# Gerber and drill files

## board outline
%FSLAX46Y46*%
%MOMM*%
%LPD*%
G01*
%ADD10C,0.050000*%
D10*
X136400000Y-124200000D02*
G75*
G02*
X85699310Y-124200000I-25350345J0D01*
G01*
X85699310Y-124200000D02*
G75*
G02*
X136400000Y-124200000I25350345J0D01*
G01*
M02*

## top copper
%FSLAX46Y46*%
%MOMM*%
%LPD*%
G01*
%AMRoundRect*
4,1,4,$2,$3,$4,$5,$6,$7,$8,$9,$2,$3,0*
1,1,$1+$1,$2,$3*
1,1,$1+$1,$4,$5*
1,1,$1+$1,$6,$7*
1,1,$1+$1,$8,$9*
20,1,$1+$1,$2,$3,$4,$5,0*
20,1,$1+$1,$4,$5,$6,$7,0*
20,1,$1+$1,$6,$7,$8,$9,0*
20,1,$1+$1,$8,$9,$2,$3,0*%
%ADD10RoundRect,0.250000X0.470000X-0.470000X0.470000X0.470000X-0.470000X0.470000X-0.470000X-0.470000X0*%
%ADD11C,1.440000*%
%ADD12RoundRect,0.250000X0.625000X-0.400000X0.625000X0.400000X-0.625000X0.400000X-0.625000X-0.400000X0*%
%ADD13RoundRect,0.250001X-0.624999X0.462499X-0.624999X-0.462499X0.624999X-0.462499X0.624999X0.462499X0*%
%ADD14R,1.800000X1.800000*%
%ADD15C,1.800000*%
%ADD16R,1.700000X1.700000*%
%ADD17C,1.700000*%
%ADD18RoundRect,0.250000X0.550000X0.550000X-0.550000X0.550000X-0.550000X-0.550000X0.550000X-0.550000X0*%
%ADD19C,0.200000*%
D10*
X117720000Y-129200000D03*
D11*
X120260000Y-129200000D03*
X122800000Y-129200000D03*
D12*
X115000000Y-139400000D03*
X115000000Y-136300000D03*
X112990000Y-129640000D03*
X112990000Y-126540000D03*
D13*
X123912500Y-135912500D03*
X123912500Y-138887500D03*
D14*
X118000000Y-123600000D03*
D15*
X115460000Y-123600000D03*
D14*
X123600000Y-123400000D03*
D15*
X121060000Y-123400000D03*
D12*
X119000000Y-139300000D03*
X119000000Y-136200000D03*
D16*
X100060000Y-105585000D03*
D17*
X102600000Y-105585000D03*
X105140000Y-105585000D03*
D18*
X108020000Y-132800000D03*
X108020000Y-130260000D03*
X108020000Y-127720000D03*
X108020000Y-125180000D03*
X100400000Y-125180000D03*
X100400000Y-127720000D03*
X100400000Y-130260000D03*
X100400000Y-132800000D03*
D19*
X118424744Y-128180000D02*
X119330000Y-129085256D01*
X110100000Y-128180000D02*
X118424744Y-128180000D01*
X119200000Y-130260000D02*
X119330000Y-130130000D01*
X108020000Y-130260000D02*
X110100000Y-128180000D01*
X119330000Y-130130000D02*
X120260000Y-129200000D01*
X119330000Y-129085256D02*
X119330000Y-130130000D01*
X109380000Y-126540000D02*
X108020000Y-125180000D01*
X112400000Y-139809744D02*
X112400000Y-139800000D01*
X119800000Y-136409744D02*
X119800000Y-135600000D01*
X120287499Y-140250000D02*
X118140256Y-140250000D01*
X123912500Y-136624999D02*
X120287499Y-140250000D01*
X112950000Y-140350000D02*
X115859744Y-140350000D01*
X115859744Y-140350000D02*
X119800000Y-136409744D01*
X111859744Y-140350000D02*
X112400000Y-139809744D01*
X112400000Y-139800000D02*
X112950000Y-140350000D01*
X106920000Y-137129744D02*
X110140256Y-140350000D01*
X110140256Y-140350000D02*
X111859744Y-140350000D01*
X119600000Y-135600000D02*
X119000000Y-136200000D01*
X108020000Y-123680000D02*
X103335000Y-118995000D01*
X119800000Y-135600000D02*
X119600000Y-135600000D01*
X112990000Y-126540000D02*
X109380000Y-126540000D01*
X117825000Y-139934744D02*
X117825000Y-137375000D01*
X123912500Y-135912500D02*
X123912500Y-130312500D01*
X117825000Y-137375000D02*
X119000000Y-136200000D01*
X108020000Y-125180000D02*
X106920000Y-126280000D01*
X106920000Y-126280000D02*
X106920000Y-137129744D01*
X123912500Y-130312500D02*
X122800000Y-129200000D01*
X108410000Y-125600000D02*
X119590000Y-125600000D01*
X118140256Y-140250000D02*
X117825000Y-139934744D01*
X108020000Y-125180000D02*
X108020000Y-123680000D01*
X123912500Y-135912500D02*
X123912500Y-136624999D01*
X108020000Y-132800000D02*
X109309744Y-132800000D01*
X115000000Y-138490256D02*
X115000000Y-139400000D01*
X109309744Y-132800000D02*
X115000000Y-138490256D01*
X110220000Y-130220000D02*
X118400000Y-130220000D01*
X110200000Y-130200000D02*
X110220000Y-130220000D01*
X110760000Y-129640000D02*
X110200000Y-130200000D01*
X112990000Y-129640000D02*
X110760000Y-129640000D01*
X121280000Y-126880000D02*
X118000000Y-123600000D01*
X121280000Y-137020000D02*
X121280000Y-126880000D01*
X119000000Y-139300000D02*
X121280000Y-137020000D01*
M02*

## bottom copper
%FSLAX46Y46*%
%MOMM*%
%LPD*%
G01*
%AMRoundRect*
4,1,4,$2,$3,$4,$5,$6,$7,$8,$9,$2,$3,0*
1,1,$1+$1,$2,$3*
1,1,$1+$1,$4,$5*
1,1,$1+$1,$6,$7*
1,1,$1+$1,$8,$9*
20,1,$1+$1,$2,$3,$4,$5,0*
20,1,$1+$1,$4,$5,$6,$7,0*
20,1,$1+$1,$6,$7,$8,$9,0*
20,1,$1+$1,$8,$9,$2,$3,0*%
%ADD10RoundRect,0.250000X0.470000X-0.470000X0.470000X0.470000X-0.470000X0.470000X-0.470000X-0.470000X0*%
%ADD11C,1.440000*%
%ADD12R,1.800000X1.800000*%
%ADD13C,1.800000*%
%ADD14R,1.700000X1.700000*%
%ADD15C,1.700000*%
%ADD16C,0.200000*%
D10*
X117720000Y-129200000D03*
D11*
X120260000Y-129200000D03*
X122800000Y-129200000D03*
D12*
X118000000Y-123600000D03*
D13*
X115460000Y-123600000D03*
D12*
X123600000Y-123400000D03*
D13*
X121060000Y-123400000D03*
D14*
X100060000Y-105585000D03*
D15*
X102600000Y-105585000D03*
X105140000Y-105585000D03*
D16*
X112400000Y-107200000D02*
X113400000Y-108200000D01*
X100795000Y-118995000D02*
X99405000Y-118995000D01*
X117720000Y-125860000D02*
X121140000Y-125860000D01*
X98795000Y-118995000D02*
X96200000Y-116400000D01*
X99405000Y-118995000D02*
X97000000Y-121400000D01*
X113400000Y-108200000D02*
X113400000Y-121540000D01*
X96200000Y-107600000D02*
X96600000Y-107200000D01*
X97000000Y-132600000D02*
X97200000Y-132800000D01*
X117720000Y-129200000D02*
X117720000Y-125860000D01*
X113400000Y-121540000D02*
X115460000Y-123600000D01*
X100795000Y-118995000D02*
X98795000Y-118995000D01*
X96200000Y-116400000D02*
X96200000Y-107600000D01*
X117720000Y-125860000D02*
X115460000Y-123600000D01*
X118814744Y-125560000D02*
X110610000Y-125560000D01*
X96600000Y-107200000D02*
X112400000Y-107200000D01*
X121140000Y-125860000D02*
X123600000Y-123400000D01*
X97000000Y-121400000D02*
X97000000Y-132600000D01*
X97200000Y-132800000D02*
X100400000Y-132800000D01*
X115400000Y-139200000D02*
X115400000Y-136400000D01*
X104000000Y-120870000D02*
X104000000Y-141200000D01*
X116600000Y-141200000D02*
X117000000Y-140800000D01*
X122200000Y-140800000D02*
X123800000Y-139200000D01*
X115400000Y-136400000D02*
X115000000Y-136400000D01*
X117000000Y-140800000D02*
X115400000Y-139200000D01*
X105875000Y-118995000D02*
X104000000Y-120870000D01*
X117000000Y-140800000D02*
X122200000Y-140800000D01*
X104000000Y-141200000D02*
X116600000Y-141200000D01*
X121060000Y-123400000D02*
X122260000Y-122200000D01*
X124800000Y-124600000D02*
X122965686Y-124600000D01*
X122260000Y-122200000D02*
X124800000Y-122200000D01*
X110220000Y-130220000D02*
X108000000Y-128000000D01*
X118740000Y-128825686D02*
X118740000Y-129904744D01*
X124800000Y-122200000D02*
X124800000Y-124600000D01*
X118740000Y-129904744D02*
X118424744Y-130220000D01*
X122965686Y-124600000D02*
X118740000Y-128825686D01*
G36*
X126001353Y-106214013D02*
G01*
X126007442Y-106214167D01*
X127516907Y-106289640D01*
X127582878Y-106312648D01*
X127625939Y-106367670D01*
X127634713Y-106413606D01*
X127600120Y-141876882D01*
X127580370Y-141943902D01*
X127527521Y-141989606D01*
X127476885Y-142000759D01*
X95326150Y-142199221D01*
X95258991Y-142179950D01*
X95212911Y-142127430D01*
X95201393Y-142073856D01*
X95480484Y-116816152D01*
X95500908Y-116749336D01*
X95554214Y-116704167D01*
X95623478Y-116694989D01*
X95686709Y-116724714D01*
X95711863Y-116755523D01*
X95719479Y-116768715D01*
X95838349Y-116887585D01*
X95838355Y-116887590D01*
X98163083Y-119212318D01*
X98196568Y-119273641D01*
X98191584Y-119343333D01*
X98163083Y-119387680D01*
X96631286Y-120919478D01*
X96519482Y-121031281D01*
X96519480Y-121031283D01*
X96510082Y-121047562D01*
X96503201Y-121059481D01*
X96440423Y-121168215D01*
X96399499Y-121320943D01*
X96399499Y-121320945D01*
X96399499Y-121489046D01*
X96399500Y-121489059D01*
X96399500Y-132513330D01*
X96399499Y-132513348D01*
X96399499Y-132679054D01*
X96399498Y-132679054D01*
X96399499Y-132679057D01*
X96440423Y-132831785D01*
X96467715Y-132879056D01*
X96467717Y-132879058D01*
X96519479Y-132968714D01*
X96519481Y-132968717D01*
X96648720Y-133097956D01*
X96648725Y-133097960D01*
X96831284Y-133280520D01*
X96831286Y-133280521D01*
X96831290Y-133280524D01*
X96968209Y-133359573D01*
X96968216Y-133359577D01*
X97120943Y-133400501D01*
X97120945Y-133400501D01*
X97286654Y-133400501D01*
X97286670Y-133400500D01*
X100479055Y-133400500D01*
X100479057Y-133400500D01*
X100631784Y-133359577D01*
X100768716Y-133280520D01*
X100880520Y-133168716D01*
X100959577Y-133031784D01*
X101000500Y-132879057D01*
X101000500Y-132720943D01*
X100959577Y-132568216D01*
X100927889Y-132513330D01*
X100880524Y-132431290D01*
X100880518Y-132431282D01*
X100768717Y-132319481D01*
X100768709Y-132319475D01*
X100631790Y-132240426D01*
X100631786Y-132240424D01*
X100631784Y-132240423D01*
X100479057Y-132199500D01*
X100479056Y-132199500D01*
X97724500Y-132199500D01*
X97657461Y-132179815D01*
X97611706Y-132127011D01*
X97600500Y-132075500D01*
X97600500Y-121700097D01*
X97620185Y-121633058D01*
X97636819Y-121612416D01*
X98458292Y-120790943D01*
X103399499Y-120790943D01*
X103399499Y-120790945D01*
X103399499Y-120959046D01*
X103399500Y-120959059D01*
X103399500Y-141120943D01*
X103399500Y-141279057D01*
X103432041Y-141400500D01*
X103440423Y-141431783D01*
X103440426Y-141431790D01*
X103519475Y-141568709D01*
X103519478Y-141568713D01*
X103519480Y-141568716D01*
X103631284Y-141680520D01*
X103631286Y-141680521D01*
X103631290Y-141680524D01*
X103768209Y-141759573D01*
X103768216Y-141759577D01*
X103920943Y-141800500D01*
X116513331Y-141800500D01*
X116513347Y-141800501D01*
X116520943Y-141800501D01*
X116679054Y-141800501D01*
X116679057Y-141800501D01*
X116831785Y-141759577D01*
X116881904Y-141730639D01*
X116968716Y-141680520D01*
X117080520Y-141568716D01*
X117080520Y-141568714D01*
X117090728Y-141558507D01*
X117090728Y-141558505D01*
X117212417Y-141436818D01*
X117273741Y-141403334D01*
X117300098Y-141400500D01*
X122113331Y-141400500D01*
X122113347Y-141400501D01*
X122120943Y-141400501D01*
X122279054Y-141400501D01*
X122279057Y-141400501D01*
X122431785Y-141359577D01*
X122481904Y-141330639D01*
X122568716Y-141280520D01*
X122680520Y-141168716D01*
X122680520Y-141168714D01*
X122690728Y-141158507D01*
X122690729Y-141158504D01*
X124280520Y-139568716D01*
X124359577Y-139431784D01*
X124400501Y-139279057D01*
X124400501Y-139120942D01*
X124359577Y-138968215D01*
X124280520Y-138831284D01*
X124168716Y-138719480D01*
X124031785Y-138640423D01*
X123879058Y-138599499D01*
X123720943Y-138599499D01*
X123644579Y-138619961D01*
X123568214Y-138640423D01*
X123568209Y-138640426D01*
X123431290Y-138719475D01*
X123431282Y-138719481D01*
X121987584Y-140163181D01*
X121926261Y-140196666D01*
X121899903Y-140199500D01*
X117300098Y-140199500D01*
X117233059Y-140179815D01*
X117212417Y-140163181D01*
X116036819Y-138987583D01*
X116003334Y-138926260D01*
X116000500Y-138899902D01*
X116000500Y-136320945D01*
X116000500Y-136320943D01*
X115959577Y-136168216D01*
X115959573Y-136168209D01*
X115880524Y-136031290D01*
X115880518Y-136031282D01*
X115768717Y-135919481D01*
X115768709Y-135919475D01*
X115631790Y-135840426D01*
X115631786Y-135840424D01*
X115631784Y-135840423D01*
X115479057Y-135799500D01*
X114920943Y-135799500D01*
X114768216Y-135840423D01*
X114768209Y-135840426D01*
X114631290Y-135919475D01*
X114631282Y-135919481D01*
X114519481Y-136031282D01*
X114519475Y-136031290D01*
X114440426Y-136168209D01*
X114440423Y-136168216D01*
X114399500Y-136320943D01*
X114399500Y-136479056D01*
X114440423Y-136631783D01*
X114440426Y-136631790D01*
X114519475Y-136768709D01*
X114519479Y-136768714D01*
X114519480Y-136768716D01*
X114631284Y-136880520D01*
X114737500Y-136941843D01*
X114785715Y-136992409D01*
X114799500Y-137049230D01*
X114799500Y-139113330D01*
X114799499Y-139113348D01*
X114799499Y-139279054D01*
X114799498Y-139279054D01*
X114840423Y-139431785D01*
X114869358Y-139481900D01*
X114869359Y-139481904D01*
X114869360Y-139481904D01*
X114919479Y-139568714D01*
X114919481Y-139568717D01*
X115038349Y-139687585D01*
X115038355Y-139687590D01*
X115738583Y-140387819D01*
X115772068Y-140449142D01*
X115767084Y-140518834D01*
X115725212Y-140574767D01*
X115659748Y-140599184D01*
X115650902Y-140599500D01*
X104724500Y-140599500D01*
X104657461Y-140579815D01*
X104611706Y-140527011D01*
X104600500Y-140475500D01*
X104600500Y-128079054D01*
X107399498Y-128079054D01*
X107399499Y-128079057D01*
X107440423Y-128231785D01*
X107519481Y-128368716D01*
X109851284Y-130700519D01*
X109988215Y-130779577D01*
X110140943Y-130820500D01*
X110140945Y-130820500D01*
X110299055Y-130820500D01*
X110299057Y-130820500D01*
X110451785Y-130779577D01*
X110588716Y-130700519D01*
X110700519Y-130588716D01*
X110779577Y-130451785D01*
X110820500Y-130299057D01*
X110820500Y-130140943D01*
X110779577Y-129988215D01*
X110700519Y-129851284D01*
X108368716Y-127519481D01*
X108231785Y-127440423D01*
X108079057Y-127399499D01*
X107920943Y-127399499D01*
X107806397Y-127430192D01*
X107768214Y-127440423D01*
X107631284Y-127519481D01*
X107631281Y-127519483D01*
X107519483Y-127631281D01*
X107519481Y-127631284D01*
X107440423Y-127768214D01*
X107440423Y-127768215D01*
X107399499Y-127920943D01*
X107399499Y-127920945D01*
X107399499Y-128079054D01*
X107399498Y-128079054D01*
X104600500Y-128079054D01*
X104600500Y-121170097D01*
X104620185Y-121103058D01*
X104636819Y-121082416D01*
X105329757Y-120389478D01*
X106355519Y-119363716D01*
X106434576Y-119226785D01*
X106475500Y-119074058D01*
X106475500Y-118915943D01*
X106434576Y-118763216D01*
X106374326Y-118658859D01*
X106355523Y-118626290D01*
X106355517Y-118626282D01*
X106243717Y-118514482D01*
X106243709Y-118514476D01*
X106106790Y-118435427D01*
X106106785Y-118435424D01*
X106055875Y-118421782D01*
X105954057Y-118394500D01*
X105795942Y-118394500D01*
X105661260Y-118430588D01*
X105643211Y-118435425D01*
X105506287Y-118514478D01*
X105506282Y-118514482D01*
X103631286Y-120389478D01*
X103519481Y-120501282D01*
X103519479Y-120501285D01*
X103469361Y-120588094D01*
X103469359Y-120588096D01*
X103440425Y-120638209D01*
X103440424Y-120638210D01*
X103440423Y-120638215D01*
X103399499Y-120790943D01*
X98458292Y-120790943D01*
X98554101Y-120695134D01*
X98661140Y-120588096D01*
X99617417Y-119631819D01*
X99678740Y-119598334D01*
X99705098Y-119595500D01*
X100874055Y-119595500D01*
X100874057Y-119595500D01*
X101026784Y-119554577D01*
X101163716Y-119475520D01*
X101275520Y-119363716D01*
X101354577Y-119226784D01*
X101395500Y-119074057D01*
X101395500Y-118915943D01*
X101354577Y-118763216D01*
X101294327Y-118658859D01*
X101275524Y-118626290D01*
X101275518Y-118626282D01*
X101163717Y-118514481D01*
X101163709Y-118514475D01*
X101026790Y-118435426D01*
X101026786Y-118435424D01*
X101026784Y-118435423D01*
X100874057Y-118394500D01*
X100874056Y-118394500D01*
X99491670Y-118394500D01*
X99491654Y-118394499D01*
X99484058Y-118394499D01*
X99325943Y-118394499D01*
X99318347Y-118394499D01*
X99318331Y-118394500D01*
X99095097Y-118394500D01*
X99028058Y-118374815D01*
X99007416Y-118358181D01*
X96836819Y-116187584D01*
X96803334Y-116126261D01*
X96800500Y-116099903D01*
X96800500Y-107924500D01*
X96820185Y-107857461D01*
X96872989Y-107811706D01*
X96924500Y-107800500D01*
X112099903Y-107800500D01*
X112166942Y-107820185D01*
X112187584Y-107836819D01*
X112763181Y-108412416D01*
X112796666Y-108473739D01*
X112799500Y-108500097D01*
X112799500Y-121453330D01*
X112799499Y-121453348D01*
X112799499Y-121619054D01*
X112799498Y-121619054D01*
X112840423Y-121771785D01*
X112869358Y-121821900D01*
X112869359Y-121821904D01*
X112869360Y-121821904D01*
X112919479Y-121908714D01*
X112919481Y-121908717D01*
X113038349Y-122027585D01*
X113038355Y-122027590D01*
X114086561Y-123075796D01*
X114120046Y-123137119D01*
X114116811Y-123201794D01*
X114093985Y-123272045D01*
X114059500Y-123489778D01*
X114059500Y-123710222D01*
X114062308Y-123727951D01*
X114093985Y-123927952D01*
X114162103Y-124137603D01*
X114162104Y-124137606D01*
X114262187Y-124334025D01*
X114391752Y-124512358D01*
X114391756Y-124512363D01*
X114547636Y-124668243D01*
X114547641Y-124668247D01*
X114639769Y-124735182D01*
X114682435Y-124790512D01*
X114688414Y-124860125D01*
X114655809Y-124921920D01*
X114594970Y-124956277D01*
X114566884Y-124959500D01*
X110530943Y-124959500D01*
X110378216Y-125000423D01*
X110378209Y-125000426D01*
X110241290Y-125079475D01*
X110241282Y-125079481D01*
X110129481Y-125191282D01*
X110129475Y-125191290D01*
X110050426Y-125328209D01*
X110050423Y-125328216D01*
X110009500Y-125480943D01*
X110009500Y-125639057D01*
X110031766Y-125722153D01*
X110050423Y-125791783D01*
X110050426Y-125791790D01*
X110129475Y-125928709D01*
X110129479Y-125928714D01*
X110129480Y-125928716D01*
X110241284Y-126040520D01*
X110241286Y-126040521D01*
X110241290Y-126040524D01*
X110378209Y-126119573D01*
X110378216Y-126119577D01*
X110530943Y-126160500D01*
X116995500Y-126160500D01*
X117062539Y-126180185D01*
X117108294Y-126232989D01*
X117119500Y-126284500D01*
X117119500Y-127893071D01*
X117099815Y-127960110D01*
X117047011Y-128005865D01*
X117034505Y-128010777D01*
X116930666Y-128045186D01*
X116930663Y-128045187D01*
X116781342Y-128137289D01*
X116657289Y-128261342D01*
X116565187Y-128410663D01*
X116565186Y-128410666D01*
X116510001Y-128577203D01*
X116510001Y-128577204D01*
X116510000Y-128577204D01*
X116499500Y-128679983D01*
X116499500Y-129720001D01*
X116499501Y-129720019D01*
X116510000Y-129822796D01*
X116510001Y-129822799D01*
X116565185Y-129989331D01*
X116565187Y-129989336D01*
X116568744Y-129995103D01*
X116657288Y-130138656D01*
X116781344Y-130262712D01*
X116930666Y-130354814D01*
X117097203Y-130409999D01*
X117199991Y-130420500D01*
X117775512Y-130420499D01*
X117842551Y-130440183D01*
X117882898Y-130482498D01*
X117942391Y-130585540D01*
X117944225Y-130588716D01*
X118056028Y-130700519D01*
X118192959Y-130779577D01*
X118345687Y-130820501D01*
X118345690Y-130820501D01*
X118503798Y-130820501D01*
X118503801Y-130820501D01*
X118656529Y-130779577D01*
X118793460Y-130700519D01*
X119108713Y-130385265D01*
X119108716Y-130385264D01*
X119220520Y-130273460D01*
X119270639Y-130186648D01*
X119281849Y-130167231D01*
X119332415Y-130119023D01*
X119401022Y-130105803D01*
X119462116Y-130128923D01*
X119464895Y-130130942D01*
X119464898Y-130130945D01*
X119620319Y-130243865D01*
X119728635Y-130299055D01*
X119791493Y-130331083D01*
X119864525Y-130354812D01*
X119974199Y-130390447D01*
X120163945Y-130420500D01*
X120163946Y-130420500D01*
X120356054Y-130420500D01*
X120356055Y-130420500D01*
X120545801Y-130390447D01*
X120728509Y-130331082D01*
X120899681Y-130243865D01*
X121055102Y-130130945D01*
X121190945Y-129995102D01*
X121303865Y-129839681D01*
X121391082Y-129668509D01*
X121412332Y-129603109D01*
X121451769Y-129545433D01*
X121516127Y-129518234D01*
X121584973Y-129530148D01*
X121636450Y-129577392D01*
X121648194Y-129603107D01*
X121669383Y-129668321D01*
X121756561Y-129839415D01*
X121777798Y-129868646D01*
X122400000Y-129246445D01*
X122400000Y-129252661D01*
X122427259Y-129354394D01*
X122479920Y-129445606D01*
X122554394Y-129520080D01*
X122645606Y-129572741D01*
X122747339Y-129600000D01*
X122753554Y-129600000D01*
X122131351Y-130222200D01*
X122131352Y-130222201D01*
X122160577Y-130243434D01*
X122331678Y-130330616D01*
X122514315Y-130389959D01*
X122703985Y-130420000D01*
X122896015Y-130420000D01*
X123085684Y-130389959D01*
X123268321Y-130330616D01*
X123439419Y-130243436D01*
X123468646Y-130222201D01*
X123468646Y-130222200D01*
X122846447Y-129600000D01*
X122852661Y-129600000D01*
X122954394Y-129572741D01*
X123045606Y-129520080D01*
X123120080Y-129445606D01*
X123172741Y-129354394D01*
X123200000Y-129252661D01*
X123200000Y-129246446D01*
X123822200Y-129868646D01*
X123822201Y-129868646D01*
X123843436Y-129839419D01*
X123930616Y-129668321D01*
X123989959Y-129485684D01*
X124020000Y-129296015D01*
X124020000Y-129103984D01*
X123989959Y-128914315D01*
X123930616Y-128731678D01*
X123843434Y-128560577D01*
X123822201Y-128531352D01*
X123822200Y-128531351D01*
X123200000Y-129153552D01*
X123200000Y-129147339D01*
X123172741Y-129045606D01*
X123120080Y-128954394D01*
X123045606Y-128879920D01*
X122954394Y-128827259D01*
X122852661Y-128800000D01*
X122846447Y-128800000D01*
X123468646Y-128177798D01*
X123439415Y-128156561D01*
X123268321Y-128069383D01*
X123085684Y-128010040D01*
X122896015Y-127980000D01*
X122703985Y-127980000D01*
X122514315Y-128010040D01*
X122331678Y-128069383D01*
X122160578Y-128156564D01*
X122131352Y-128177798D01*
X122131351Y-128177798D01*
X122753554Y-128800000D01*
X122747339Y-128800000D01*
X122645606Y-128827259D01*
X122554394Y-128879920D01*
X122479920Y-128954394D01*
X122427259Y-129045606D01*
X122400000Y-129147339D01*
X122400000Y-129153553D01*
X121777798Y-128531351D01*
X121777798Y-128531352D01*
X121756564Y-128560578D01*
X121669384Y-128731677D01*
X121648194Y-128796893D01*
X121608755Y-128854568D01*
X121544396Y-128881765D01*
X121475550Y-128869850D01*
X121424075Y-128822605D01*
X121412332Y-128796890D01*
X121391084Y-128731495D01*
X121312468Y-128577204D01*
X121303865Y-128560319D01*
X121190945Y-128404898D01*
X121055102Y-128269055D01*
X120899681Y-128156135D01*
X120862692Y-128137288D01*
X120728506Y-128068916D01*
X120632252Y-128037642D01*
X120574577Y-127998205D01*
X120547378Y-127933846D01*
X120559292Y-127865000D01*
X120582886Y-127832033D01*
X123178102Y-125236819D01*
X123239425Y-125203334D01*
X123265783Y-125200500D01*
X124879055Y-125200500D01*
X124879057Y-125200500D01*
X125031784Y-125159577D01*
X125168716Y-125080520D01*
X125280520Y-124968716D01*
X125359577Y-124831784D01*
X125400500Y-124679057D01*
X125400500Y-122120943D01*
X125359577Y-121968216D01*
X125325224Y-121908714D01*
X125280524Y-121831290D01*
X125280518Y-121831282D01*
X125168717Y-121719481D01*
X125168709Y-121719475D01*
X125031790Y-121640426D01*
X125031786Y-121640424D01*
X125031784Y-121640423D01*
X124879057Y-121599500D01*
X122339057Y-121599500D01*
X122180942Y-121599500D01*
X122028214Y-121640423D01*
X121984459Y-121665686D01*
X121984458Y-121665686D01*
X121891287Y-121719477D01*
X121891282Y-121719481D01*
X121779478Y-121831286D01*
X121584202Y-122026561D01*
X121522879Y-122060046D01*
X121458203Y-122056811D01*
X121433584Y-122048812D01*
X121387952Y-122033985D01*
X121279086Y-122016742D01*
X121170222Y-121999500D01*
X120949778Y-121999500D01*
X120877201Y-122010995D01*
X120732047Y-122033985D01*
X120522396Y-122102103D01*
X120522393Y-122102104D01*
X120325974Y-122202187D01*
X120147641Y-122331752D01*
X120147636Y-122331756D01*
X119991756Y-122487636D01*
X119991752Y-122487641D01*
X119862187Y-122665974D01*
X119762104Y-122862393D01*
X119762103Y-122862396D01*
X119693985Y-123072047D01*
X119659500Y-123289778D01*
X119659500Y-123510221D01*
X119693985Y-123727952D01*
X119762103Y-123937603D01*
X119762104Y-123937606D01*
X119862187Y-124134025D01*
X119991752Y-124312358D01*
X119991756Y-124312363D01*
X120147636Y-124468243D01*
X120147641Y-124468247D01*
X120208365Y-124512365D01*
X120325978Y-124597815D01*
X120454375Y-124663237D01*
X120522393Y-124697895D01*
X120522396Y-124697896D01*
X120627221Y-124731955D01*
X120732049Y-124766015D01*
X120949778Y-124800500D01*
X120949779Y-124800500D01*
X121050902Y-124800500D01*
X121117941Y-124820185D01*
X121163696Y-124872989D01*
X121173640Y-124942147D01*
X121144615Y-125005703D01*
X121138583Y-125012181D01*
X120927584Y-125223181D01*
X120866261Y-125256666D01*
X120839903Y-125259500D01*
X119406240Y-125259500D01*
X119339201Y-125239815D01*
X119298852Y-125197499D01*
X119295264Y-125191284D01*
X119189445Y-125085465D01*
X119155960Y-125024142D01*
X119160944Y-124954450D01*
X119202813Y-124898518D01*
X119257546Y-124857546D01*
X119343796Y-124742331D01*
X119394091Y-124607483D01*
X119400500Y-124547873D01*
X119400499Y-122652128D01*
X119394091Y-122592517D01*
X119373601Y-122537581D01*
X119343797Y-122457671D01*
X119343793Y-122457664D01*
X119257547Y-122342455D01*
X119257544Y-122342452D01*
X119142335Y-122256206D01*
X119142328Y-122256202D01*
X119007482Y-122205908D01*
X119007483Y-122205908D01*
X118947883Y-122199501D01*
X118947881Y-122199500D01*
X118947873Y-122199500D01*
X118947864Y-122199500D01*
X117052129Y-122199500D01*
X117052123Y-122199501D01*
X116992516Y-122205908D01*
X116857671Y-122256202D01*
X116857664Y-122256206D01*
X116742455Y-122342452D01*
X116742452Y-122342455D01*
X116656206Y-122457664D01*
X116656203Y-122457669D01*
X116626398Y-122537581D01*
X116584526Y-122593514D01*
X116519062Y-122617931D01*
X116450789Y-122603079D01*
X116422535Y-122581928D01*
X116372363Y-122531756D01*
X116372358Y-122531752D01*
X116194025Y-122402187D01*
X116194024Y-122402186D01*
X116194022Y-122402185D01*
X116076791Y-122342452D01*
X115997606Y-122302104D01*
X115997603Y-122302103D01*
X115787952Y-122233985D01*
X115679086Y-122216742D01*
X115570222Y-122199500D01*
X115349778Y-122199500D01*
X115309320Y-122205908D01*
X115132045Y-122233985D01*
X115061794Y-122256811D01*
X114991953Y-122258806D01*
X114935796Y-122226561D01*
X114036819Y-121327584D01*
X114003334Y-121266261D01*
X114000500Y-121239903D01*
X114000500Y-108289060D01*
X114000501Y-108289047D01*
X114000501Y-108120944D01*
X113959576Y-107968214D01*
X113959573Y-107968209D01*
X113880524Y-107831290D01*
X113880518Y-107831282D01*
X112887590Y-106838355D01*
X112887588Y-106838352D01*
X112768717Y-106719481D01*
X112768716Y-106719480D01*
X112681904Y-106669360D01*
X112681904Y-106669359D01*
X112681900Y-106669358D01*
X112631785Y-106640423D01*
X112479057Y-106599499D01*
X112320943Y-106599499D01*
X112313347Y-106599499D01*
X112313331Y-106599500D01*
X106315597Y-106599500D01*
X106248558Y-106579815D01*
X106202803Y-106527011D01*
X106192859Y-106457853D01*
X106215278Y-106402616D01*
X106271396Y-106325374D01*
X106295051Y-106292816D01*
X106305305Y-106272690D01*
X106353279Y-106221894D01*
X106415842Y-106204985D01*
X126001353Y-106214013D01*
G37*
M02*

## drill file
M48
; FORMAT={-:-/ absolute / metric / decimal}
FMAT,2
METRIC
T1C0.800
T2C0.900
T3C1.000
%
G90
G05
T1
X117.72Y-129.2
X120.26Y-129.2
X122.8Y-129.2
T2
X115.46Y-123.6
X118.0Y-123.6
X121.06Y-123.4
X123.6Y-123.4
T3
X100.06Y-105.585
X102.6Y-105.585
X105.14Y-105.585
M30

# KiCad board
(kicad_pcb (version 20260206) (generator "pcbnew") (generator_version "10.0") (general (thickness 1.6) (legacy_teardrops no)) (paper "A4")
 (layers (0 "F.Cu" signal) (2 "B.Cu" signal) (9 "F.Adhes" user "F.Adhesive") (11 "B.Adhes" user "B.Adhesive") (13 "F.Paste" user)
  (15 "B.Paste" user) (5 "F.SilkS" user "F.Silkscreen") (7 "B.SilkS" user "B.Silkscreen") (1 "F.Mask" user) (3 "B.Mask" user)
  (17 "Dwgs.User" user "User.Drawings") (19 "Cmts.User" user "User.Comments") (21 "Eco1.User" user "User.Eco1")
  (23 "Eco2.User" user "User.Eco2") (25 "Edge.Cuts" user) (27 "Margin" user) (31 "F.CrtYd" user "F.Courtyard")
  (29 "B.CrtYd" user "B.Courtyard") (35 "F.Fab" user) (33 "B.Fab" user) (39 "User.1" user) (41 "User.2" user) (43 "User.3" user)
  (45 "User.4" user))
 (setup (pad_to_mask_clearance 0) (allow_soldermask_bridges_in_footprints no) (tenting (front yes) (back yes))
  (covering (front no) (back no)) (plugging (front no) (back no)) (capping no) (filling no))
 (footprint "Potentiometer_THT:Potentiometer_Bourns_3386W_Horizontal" (layer "F.Cu") (at 117.72 129.2)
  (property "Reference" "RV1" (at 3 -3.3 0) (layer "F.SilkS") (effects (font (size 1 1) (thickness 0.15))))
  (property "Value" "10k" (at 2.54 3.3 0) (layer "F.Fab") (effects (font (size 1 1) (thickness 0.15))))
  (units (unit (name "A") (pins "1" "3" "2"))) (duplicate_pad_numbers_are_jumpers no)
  (pad "1" thru_hole roundrect (at 0 0 90) (size 1.44 1.44) (drill 0.8) (layers "*.Cu" "*.Mask") (remove_unused_layers no)
   (roundrect_rratio 0.1736111111) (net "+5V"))
  (pad "2" thru_hole circle (at 2.54 0 90) (size 1.44 1.44) (drill 0.8) (layers "*.Cu" "*.Mask") (remove_unused_layers no)
   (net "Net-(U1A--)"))
  (pad "3" thru_hole circle (at 5.08 0 90) (size 1.44 1.44) (drill 0.8) (layers "*.Cu" "*.Mask") (remove_unused_layers no) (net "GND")))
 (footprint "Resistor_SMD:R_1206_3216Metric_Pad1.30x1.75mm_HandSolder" (layer "F.Cu") (at 115 137.85 90)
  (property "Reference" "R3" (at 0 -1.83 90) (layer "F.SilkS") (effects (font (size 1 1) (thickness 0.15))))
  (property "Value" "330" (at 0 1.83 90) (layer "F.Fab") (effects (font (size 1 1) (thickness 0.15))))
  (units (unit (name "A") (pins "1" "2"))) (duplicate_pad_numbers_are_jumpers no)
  (pad "1" smd roundrect (at -1.55 0 90) (size 1.3 1.75) (layers "F.Cu" "F.Mask" "F.Paste") (roundrect_rratio 0.192308)
   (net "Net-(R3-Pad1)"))
  (pad "2" smd roundrect (at 1.55 0 90) (size 1.3 1.75) (layers "F.Cu" "F.Mask" "F.Paste") (roundrect_rratio 0.192308) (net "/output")))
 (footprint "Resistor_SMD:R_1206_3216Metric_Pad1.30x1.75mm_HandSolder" (layer "F.Cu") (at 112.99 128.09 90)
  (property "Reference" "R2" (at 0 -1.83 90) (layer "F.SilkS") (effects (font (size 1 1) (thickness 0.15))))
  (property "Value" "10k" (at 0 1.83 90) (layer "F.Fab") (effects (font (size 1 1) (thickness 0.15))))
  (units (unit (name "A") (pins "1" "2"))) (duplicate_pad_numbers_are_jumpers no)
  (pad "1" smd roundrect (at -1.55 0 90) (size 1.3 1.75) (layers "F.Cu" "F.Mask" "F.Paste") (roundrect_rratio 0.192308) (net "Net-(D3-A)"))
  (pad "2" smd roundrect (at 1.55 0 90) (size 1.3 1.75) (layers "F.Cu" "F.Mask" "F.Paste") (roundrect_rratio 0.192308) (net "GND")))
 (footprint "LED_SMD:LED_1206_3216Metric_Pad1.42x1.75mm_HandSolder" (layer "F.Cu") (at 123.9125 137.4 -90)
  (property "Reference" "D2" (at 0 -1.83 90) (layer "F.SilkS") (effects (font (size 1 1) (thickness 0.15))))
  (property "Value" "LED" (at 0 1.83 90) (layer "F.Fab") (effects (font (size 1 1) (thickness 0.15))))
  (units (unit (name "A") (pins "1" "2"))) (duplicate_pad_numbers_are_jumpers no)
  (pad "1" smd roundrect (at -1.4875 0 270) (size 1.425 1.75) (layers "F.Cu" "F.Mask" "F.Paste") (roundrect_rratio 0.175439) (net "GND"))
  (pad "2" smd roundrect (at 1.4875 0 270) (size 1.425 1.75) (layers "F.Cu" "F.Mask" "F.Paste") (roundrect_rratio 0.175439) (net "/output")))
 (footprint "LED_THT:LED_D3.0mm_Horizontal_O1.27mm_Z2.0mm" (layer "F.Cu") (at 118 123.6 180)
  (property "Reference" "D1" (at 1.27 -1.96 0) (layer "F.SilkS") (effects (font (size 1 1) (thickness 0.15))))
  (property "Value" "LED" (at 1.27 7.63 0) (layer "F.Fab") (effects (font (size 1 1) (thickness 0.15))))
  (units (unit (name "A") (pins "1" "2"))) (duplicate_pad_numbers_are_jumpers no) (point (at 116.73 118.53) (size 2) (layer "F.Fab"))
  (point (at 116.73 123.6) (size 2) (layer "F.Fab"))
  (pad "1" thru_hole rect (at 0 0 180) (size 1.8 1.8) (drill 0.9) (layers "*.Cu" "*.Mask") (remove_unused_layers no) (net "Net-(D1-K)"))
  (pad "2" thru_hole circle (at 2.54 0 180) (size 1.8 1.8) (drill 0.9) (layers "*.Cu" "*.Mask") (remove_unused_layers no) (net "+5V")))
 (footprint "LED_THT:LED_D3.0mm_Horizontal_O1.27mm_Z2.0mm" (layer "F.Cu") (at 123.6 123.4 180)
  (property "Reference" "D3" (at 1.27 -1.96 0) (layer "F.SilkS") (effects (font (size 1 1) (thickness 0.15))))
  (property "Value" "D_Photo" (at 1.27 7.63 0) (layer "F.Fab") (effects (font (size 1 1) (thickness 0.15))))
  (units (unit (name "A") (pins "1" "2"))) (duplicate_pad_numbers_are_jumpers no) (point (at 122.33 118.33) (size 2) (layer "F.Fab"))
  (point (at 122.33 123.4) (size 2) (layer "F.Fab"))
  (pad "1" thru_hole rect (at 0 0 180) (size 1.8 1.8) (drill 0.9) (layers "*.Cu" "*.Mask") (remove_unused_layers no) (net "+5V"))
  (pad "2" thru_hole circle (at 2.54 0 180) (size 1.8 1.8) (drill 0.9) (layers "*.Cu" "*.Mask") (remove_unused_layers no) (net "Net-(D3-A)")))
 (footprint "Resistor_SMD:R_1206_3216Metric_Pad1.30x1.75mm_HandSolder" (layer "F.Cu") (at 119 137.75 90)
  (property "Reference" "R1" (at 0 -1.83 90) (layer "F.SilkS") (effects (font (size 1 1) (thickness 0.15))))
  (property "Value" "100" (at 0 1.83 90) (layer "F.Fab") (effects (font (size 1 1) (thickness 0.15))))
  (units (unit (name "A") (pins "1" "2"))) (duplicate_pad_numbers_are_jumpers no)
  (pad "1" smd roundrect (at -1.55 0 90) (size 1.3 1.75) (layers "F.Cu" "F.Mask" "F.Paste") (roundrect_rratio 0.192308) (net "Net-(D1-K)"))
  (pad "2" smd roundrect (at 1.55 0 90) (size 1.3 1.75) (layers "F.Cu" "F.Mask" "F.Paste") (roundrect_rratio 0.192308) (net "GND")))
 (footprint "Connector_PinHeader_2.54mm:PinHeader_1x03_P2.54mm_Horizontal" (layer "F.Cu") (at 100.06 105.585 90)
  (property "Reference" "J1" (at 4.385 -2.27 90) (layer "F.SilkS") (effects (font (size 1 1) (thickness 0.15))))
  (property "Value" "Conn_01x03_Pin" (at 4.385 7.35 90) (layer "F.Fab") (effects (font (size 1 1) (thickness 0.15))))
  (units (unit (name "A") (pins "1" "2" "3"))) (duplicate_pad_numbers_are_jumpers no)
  (pad "1" thru_hole rect (at 0 0 90) (size 1.7 1.7) (drill 1) (layers "*.Cu" "*.Mask") (remove_unused_layers no) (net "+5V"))
  (pad "2" thru_hole circle (at 0 2.54 90) (size 1.7 1.7) (drill 1) (layers "*.Cu" "*.Mask") (remove_unused_layers no) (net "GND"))
  (pad "3" thru_hole circle (at 0 5.08 90) (size 1.7 1.7) (drill 1) (layers "*.Cu" "*.Mask") (remove_unused_layers no) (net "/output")))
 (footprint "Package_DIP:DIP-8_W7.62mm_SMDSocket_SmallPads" (layer "F.Cu") (at 104.21 128.99 180)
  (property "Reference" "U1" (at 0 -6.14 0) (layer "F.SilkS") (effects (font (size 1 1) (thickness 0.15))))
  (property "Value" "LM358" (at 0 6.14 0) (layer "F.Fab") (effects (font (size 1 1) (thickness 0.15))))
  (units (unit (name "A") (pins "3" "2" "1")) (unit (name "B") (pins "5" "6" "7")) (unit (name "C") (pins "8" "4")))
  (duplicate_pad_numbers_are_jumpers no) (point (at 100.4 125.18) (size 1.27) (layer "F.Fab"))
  (pad "1" smd roundrect (at -3.81 -3.81 180) (size 1.6 1.6) (layers "F.Cu" "F.Mask" "F.Paste") (roundrect_rratio 0.15625)
   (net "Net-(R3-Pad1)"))
  (pad "2" smd roundrect (at -3.81 -1.27 180) (size 1.6 1.6) (layers "F.Cu" "F.Mask" "F.Paste") (roundrect_rratio 0.15625)
   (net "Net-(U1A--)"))
  (pad "3" smd roundrect (at -3.81 1.27 180) (size 1.6 1.6) (layers "F.Cu" "F.Mask" "F.Paste") (roundrect_rratio 0.15625) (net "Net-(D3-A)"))
  (pad "4" smd roundrect (at -3.81 3.81 180) (size 1.6 1.6) (layers "F.Cu" "F.Mask" "F.Paste") (roundrect_rratio 0.15625) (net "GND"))
  (pad "5" smd roundrect (at 3.81 3.81 180) (size 1.6 1.6) (layers "F.Cu" "F.Mask" "F.Paste") (roundrect_rratio 0.15625))
  (pad "6" smd roundrect (at 3.81 1.27 180) (size 1.6 1.6) (layers "F.Cu" "F.Mask" "F.Paste") (roundrect_rratio 0.15625))
  (pad "7" smd roundrect (at 3.81 -1.27 180) (size 1.6 1.6) (layers "F.Cu" "F.Mask" "F.Paste") (roundrect_rratio 0.15625))
  (pad "8" smd roundrect (at 3.81 -3.81 180) (size 1.6 1.6) (layers "F.Cu" "F.Mask" "F.Paste") (roundrect_rratio 0.15625) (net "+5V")))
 (gr_circle (center 111.049655 124.2) (end 132.049655 138.4) (stroke (width 0.05) (type default)) (fill no) (layer "Edge.Cuts"))
 (segment (start 112.4 107.2) (end 113.4 108.2) (width 0.2) (layer "B.Cu") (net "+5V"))
 (segment (start 100.795 118.995) (end 99.405 118.995) (width 0.2) (layer "B.Cu") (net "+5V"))
 (segment (start 117.72 125.86) (end 121.14 125.86) (width 0.2) (layer "B.Cu") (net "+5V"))
 (segment (start 98.795 118.995) (end 96.2 116.4) (width 0.2) (layer "B.Cu") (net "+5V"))
 (segment (start 99.405 118.995) (end 97 121.4) (width 0.2) (layer "B.Cu") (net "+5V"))
 (segment (start 113.4 108.2) (end 113.4 121.54) (width 0.2) (layer "B.Cu") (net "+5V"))
 (segment (start 96.2 107.6) (end 96.6 107.2) (width 0.2) (layer "B.Cu") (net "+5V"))
 (segment (start 97 132.6) (end 97.2 132.8) (width 0.2) (layer "B.Cu") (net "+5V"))
 (segment (start 117.72 129.2) (end 117.72 125.86) (width 0.2) (layer "B.Cu") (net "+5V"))
 (segment (start 113.4 121.54) (end 115.46 123.6) (width 0.2) (layer "B.Cu") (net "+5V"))
 (segment (start 100.795 118.995) (end 98.795 118.995) (width 0.2) (layer "B.Cu") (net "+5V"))
 (segment (start 96.2 116.4) (end 96.2 107.6) (width 0.2) (layer "B.Cu") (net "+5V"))
 (segment (start 117.72 125.86) (end 115.46 123.6) (width 0.2) (layer "B.Cu") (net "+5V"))
 (segment (start 118.814744 125.56) (end 110.61 125.56) (width 0.2) (layer "B.Cu") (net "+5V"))
 (segment (start 96.6 107.2) (end 112.4 107.2) (width 0.2) (layer "B.Cu") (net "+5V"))
 (segment (start 121.14 125.86) (end 123.6 123.4) (width 0.2) (layer "B.Cu") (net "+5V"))
 (segment (start 97 121.4) (end 97 132.6) (width 0.2) (layer "B.Cu") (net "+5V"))
 (segment (start 97.2 132.8) (end 100.4 132.8) (width 0.2) (layer "B.Cu") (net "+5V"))
 (segment (start 118.424744 128.18) (end 119.33 129.085256) (width 0.2) (layer "F.Cu") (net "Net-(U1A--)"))
 (segment (start 110.1 128.18) (end 118.424744 128.18) (width 0.2) (layer "F.Cu") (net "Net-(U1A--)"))
 (segment (start 119.2 130.26) (end 119.33 130.13) (width 0.2) (layer "F.Cu") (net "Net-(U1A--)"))
 (segment (start 108.02 130.26) (end 110.1 128.18) (width 0.2) (layer "F.Cu") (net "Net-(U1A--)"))
 (segment (start 119.33 130.13) (end 120.26 129.2) (width 0.2) (layer "F.Cu") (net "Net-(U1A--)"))
 (segment (start 119.33 129.085256) (end 119.33 130.13) (width 0.2) (layer "F.Cu") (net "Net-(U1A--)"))
 (segment (start 109.38 126.54) (end 108.02 125.18) (width 0.2) (layer "F.Cu") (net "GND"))
 (segment (start 112.4 139.809744) (end 112.4 139.8) (width 0.2) (layer "F.Cu") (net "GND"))
 (segment (start 119.8 136.409744) (end 119.8 135.6) (width 0.2) (layer "F.Cu") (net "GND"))
 (segment (start 120.287499 140.25) (end 118.140256 140.25) (width 0.2) (layer "F.Cu") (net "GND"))
 (segment (start 123.9125 136.624999) (end 120.287499 140.25) (width 0.2) (layer "F.Cu") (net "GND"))
 (segment (start 112.95 140.35) (end 115.859744 140.35) (width 0.2) (layer "F.Cu") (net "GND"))
 (segment (start 115.859744 140.35) (end 119.8 136.409744) (width 0.2) (layer "F.Cu") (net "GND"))
 (segment (start 111.859744 140.35) (end 112.4 139.809744) (width 0.2) (layer "F.Cu") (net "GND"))
 (segment (start 112.4 139.8) (end 112.95 140.35) (width 0.2) (layer "F.Cu") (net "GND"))
 (segment (start 106.92 137.129744) (end 110.140256 140.35) (width 0.2) (layer "F.Cu") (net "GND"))
 (segment (start 110.140256 140.35) (end 111.859744 140.35) (width 0.2) (layer "F.Cu") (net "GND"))
 (segment (start 119.6 135.6) (end 119 136.2) (width 0.2) (layer "F.Cu") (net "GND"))
 (segment (start 108.02 123.68) (end 103.335 118.995) (width 0.2) (layer "F.Cu") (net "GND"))
 (segment (start 119.8 135.6) (end 119.6 135.6) (width 0.2) (layer "F.Cu") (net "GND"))
 (segment (start 112.99 126.54) (end 109.38 126.54) (width 0.2) (layer "F.Cu") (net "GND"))
 (segment (start 117.825 139.934744) (end 117.825 137.375) (width 0.2) (layer "F.Cu") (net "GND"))
 (segment (start 123.9125 135.9125) (end 123.9125 130.3125) (width 0.2) (layer "F.Cu") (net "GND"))
 (segment (start 117.825 137.375) (end 119 136.2) (width 0.2) (layer "F.Cu") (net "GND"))
 (segment (start 108.02 125.18) (end 106.92 126.28) (width 0.2) (layer "F.Cu") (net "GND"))
 (segment (start 106.92 126.28) (end 106.92 137.129744) (width 0.2) (layer "F.Cu") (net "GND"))
 (segment (start 123.9125 130.3125) (end 122.8 129.2) (width 0.2) (layer "F.Cu") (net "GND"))
 (segment (start 108.41 125.6) (end 119.59 125.6) (width 0.2) (layer "F.Cu") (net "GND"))
 (segment (start 118.140256 140.25) (end 117.825 139.934744) (width 0.2) (layer "F.Cu") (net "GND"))
 (segment (start 108.02 125.18) (end 108.02 123.68) (width 0.2) (layer "F.Cu") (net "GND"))
 (segment (start 123.9125 135.9125) (end 123.9125 136.624999) (width 0.2) (layer "F.Cu") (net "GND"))
 (segment (start 108.02 132.8) (end 109.309744 132.8) (width 0.2) (layer "F.Cu") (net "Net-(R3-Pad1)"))
 (segment (start 115 138.490256) (end 115 139.4) (width 0.2) (layer "F.Cu") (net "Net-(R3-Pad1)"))
 (segment (start 109.309744 132.8) (end 115 138.490256) (width 0.2) (layer "F.Cu") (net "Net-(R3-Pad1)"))
 (segment (start 115.4 139.2) (end 115.4 136.4) (width 0.2) (layer "B.Cu") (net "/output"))
 (segment (start 104 120.87) (end 104 141.2) (width 0.2) (layer "B.Cu") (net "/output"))
 (segment (start 116.6 141.2) (end 117 140.8) (width 0.2) (layer "B.Cu") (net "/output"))
 (segment (start 122.2 140.8) (end 123.8 139.2) (width 0.2) (layer "B.Cu") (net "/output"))
 (segment (start 115.4 136.4) (end 115 136.4) (width 0.2) (layer "B.Cu") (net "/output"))
 (segment (start 117 140.8) (end 115.4 139.2) (width 0.2) (layer "B.Cu") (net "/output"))
 (segment (start 105.875 118.995) (end 104 120.87) (width 0.2) (layer "B.Cu") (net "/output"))
 (segment (start 117 140.8) (end 122.2 140.8) (width 0.2) (layer "B.Cu") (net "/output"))
 (segment (start 104 141.2) (end 116.6 141.2) (width 0.2) (layer "B.Cu") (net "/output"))
 (segment (start 110.22 130.22) (end 118.4 130.22) (width 0.2) (layer "F.Cu") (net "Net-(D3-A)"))
 (segment (start 110.2 130.2) (end 110.22 130.22) (width 0.2) (layer "F.Cu") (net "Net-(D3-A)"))
 (segment (start 110.76 129.64) (end 110.2 130.2) (width 0.2) (layer "F.Cu") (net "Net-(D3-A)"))
 (segment (start 112.99 129.64) (end 110.76 129.64) (width 0.2) (layer "F.Cu") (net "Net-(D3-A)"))
 (segment (start 121.06 123.4) (end 122.26 122.2) (width 0.2) (layer "B.Cu") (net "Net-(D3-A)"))
 (segment (start 124.8 124.6) (end 122.965686 124.6) (width 0.2) (layer "B.Cu") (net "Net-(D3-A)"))
 (segment (start 122.26 122.2) (end 124.8 122.2) (width 0.2) (layer "B.Cu") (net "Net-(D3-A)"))
 (segment (start 110.22 130.22) (end 108 128) (width 0.2) (layer "B.Cu") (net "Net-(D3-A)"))
 (segment (start 118.74 128.825686) (end 118.74 129.904744) (width 0.2) (layer "B.Cu") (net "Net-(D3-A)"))
 (segment (start 124.8 122.2) (end 124.8 124.6) (width 0.2) (layer "B.Cu") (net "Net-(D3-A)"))
 (segment (start 118.74 129.904744) (end 118.424744 130.22) (width 0.2) (layer "B.Cu") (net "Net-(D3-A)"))
 (segment (start 122.965686 124.6) (end 118.74 128.825686) (width 0.2) (layer "B.Cu") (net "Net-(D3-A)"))
 (segment (start 121.28 126.88) (end 118 123.6) (width 0.2) (layer "F.Cu") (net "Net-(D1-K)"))
 (segment (start 121.28 137.02) (end 121.28 126.88) (width 0.2) (layer "F.Cu") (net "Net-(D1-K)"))
 (segment (start 119 139.3) (end 121.28 137.02) (width 0.2) (layer "F.Cu") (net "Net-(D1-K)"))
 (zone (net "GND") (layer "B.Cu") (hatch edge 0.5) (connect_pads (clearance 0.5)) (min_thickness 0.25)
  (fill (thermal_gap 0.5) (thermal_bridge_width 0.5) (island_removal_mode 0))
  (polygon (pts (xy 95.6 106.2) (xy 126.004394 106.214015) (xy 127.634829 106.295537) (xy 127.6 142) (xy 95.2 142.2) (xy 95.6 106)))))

